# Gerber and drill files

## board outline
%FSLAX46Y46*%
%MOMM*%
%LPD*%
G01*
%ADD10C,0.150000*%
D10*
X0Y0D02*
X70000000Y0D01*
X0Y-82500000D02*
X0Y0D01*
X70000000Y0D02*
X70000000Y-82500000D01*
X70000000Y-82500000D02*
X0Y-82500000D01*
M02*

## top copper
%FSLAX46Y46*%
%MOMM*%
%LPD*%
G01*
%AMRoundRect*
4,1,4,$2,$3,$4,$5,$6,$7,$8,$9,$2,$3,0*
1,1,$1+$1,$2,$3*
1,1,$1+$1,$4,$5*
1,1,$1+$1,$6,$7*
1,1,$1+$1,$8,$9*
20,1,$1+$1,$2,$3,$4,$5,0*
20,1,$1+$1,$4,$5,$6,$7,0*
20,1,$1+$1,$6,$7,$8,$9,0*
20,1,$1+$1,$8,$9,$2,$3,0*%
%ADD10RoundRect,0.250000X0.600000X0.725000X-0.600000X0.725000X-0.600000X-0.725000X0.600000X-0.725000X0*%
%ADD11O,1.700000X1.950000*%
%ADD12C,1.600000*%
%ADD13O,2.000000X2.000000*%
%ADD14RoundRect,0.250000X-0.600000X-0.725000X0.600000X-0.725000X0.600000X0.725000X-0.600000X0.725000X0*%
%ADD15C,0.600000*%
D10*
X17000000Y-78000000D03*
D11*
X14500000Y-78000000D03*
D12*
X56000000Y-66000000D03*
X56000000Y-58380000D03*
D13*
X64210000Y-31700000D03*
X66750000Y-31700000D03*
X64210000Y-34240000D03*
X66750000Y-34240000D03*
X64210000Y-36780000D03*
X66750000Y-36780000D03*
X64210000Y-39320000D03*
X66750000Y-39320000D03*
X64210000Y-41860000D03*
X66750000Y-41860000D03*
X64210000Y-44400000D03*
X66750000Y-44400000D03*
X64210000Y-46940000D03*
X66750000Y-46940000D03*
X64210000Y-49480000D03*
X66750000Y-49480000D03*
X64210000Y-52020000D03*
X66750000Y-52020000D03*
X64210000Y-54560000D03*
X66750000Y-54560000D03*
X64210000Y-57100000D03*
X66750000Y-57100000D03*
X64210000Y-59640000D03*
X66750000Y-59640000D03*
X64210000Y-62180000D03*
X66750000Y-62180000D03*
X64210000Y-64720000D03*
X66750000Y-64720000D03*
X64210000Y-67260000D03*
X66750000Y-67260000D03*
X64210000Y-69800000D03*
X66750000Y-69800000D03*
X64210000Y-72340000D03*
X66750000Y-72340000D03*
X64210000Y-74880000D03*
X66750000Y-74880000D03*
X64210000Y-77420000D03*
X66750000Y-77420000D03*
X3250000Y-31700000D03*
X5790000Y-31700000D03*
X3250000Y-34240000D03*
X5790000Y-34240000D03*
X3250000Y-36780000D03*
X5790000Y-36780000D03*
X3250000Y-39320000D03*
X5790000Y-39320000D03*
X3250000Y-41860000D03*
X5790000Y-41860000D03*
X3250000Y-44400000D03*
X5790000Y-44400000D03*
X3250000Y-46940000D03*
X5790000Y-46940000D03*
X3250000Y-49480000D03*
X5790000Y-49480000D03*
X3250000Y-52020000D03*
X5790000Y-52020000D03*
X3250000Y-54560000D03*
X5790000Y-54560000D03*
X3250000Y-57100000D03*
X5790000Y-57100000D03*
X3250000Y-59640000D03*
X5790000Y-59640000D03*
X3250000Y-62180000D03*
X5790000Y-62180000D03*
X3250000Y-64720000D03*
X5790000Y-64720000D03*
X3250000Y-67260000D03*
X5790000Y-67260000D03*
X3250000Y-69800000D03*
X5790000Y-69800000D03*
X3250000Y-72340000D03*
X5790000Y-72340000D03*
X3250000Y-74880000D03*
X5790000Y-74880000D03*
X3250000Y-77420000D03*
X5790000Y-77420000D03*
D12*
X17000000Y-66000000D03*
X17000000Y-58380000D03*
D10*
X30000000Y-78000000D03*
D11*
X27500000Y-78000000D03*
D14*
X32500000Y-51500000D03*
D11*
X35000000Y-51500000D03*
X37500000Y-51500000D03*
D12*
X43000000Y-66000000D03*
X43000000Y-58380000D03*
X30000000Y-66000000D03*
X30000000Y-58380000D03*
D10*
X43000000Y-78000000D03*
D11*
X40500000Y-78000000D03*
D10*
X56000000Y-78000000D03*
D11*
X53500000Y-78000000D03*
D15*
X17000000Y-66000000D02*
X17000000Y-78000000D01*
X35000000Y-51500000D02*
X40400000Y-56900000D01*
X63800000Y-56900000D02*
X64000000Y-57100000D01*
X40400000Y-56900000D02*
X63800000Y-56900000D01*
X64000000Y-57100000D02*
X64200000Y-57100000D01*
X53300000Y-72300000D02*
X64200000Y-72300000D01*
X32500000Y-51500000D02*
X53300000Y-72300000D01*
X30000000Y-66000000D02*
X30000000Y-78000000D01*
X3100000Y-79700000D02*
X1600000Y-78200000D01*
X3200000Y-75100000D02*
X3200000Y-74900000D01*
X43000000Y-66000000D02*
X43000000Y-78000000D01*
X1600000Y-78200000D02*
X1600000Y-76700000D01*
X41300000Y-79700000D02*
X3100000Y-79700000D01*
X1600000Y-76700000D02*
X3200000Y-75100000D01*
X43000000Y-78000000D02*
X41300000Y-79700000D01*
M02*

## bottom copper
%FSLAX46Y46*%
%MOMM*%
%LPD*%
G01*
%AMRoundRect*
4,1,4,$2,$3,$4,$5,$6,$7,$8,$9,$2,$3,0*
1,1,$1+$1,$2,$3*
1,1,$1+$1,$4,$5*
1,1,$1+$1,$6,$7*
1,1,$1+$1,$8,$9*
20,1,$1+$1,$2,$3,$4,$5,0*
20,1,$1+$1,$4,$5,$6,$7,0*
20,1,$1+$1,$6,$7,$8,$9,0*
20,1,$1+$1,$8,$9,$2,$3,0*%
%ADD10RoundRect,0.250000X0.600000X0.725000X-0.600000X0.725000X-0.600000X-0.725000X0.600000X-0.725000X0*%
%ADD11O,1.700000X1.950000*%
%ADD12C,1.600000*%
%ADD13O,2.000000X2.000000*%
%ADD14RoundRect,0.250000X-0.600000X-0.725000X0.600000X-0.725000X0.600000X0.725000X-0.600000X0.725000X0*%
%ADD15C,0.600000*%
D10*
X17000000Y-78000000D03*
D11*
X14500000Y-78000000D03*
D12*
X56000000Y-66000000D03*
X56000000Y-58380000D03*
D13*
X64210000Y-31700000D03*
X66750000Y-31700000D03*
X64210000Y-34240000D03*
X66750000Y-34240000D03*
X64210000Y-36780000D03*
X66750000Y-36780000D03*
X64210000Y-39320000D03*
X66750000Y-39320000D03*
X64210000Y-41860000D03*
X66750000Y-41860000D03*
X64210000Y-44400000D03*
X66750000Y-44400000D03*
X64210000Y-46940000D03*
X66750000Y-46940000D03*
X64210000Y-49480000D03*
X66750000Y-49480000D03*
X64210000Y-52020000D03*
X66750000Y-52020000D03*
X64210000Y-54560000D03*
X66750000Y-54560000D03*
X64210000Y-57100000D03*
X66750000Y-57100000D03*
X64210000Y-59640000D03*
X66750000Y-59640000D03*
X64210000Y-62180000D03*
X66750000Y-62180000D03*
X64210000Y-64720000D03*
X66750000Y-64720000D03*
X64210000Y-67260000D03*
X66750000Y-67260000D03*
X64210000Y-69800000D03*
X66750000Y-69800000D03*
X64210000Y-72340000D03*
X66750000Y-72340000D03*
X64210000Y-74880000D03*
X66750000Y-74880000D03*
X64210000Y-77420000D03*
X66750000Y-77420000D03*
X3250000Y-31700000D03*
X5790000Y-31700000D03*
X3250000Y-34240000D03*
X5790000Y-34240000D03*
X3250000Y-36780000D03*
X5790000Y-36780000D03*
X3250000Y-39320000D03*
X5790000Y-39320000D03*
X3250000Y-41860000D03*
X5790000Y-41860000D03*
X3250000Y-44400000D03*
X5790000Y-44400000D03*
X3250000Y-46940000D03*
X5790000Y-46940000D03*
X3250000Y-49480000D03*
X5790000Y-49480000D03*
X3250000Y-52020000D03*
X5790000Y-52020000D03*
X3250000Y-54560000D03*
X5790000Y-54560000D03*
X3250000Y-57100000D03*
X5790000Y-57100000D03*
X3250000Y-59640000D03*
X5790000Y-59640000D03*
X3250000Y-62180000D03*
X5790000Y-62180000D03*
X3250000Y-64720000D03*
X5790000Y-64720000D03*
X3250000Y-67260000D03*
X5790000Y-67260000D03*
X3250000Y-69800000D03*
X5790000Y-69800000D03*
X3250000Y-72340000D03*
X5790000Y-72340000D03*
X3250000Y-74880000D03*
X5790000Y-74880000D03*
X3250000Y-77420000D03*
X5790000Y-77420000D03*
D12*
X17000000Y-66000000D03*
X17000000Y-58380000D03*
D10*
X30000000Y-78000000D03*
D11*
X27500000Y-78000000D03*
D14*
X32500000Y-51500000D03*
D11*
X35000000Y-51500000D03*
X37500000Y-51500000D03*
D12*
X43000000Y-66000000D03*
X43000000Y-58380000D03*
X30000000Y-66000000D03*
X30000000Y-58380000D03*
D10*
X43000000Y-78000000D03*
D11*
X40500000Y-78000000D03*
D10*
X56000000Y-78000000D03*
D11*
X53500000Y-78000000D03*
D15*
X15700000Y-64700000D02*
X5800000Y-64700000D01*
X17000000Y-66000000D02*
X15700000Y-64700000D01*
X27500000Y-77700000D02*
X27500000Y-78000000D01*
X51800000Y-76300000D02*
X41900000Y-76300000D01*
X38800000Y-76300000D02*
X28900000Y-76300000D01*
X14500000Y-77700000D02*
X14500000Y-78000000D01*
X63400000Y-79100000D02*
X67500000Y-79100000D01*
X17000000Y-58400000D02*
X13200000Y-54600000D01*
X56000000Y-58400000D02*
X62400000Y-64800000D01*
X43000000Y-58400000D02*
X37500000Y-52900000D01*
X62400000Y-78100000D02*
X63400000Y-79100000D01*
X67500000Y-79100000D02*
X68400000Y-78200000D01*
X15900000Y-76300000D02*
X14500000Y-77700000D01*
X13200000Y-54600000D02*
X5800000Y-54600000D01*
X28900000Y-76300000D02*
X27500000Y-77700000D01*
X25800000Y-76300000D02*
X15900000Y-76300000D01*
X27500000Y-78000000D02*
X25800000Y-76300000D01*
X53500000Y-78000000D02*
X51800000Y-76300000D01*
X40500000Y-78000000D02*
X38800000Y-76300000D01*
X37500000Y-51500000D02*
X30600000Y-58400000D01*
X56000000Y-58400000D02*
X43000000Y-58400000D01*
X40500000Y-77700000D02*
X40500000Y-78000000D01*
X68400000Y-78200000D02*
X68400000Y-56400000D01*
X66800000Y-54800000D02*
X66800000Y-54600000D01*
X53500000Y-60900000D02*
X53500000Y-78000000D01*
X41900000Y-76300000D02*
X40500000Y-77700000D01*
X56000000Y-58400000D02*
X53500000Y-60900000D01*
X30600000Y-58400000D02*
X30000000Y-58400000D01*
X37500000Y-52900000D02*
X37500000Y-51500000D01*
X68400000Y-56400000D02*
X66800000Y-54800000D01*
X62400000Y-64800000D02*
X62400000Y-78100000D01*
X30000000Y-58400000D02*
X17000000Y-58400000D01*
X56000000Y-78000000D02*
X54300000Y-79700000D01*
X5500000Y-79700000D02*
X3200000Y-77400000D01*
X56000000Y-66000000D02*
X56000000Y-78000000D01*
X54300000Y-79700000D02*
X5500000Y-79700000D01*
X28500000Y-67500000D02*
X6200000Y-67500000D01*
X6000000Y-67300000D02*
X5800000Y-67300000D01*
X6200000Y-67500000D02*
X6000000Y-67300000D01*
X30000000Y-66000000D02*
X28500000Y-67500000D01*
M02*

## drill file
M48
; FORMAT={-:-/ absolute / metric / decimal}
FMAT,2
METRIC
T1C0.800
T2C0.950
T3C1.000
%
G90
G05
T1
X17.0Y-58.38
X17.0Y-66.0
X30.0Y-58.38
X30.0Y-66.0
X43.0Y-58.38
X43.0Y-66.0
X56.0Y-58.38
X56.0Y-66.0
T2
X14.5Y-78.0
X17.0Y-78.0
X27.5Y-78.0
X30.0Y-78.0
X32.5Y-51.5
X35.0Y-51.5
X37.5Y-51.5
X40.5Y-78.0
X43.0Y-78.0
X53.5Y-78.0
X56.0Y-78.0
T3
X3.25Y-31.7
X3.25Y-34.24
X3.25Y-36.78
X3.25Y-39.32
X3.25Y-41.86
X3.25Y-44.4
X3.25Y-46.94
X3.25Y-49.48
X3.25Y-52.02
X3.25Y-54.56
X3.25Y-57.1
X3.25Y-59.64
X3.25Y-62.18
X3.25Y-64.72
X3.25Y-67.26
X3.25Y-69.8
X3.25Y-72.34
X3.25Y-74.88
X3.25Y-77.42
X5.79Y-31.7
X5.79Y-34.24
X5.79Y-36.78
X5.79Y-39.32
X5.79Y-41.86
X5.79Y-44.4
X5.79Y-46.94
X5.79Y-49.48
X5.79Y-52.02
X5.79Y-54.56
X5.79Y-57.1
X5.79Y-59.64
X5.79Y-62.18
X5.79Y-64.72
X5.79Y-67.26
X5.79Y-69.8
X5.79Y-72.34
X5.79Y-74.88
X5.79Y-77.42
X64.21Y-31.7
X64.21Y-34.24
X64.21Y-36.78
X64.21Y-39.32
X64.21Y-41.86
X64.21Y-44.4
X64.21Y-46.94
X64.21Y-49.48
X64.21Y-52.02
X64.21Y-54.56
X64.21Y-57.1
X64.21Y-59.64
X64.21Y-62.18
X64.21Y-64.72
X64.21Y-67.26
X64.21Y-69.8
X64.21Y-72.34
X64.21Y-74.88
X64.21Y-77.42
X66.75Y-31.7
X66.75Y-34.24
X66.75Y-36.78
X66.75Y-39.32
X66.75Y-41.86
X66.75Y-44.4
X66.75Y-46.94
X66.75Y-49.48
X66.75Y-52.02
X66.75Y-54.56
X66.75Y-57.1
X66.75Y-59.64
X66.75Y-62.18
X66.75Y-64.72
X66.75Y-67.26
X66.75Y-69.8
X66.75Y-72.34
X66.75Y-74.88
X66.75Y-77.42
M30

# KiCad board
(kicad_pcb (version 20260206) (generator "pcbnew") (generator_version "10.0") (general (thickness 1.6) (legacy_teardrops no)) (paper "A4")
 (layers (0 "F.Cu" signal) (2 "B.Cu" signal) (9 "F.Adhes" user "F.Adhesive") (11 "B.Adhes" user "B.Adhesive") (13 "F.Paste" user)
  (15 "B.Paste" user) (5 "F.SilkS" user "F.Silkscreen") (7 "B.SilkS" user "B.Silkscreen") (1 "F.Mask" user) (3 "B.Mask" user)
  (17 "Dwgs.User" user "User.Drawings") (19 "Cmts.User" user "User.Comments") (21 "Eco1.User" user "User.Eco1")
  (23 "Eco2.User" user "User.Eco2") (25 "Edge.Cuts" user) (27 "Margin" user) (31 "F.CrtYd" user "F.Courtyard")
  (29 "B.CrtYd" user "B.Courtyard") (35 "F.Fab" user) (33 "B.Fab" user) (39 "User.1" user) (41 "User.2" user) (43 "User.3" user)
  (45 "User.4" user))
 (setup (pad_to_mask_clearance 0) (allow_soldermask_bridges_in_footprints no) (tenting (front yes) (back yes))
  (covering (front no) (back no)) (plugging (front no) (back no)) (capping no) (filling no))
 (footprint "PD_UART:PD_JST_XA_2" (layer "F.Cu") (at 17 78 180)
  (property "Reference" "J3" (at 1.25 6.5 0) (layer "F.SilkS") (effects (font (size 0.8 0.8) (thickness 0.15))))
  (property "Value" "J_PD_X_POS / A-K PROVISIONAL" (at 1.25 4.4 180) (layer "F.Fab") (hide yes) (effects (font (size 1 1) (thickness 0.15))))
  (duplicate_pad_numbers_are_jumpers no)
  (pad "1" thru_hole roundrect (at 0 0 180) (size 1.7 1.95) (drill 0.95) (layers "*.Cu" "*.Mask") (remove_unused_layers no)
   (roundrect_rratio 0.147059) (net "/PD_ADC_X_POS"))
  (pad "2" thru_hole oval (at 2.5 0 180) (size 1.7 1.95) (drill 0.95) (layers "*.Cu" "*.Mask") (remove_unused_layers no) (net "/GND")))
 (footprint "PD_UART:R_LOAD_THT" (layer "F.Cu") (at 56 66 90)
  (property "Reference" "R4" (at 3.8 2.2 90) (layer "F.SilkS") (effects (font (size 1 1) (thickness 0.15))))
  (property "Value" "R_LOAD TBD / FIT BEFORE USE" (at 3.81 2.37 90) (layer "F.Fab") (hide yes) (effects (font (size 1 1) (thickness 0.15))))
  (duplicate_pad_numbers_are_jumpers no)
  (pad "1" thru_hole circle (at 0 0 90) (size 1.6 1.6) (drill 0.8) (layers "*.Cu" "*.Mask") (remove_unused_layers no) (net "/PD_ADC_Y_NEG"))
  (pad "2" thru_hole circle (at 7.62 0 90) (size 1.6 1.6) (drill 0.8) (layers "*.Cu" "*.Mask") (remove_unused_layers no) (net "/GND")))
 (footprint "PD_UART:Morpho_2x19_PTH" (layer "F.Cu") (at 64.21 31.7)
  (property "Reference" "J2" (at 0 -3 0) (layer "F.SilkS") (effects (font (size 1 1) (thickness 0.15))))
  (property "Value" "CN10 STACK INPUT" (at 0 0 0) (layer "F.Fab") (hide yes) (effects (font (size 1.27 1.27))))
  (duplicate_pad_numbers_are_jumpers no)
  (pad "1" thru_hole oval (at 0 0) (size 2 2) (drill 1) (layers "*.Cu") (remove_unused_layers no) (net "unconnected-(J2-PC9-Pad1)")
   (thermal_bridge_angle 45))
  (pad "2" thru_hole oval (at 2.54 0) (size 2 2) (drill 1) (layers "*.Cu") (remove_unused_layers no) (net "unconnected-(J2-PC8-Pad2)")
   (thermal_bridge_angle 45))
  (pad "3" thru_hole oval (at 0 2.54) (size 2 2) (drill 1) (layers "*.Cu") (remove_unused_layers no) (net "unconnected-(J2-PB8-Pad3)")
   (thermal_bridge_angle 45))
  (pad "4" thru_hole oval (at 2.54 2.54) (size 2 2) (drill 1) (layers "*.Cu") (remove_unused_layers no) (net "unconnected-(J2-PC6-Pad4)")
   (thermal_bridge_angle 45))
  (pad "5" thru_hole oval (at 0 5.08) (size 2 2) (drill 1) (layers "*.Cu") (remove_unused_layers no) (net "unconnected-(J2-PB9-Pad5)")
   (thermal_bridge_angle 45))
  (pad "6" thru_hole oval (at 2.54 5.08) (size 2 2) (drill 1) (layers "*.Cu") (remove_unused_layers no) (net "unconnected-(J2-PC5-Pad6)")
   (thermal_bridge_angle 45))
  (pad "7" thru_hole oval (at 0 7.62) (size 2 2) (drill 1) (layers "*.Cu") (remove_unused_layers no) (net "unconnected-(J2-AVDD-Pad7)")
   (thermal_bridge_angle 45))
  (pad "8" thru_hole oval (at 2.54 7.62) (size 2 2) (drill 1) (layers "*.Cu") (remove_unused_layers no) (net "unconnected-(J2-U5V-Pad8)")
   (thermal_bridge_angle 45))
  (pad "9" thru_hole oval (at 0 10.16) (size 2 2) (drill 1) (layers "*.Cu") (remove_unused_layers no) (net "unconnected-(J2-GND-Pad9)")
   (thermal_bridge_angle 45))
  (pad "10" thru_hole oval (at 2.54 10.16) (size 2 2) (drill 1) (layers "*.Cu") (remove_unused_layers no) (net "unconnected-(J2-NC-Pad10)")
   (thermal_bridge_angle 45))
  (pad "11" thru_hole oval (at 0 12.7) (size 2 2) (drill 1) (layers "*.Cu") (remove_unused_layers no) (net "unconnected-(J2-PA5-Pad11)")
   (thermal_bridge_angle 45))
  (pad "12" thru_hole oval (at 2.54 12.7) (size 2 2) (drill 1) (layers "*.Cu") (remove_unused_layers no) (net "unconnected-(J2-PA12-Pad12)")
   (thermal_bridge_angle 45))
  (pad "13" thru_hole oval (at 0 15.24) (size 2 2) (drill 1) (layers "*.Cu") (remove_unused_layers no) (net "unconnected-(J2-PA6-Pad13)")
   (thermal_bridge_angle 45))
  (pad "14" thru_hole oval (at 2.54 15.24) (size 2 2) (drill 1) (layers "*.Cu") (remove_unused_layers no)
   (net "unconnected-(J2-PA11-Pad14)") (thermal_bridge_angle 45))
  (pad "15" thru_hole oval (at 0 17.78) (size 2 2) (drill 1) (layers "*.Cu") (remove_unused_layers no) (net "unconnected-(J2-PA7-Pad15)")
   (thermal_bridge_angle 45))
  (pad "16" thru_hole oval (at 2.54 17.78) (size 2 2) (drill 1) (layers "*.Cu") (remove_unused_layers no)
   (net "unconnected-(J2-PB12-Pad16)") (thermal_bridge_angle 45))
  (pad "17" thru_hole oval (at 0 20.32) (size 2 2) (drill 1) (layers "*.Cu") (remove_unused_layers no) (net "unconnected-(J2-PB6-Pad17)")
   (thermal_bridge_angle 45))
  (pad "18" thru_hole oval (at 2.54 20.32) (size 2 2) (drill 1) (layers "*.Cu") (remove_unused_layers no)
   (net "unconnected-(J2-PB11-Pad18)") (thermal_bridge_angle 45))
  (pad "19" thru_hole oval (at 0 22.86) (size 2 2) (drill 1) (layers "*.Cu") (remove_unused_layers no) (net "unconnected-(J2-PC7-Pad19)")
   (thermal_bridge_angle 45))
  (pad "20" thru_hole oval (at 2.54 22.86) (size 2 2) (drill 1) (layers "*.Cu") (remove_unused_layers no) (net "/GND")
   (thermal_bridge_angle 45))
  (pad "21" thru_hole oval (at 0 25.4) (size 2 2) (drill 1) (layers "*.Cu") (remove_unused_layers no) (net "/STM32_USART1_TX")
   (thermal_bridge_angle 45))
  (pad "22" thru_hole oval (at 2.54 25.4) (size 2 2) (drill 1) (layers "*.Cu") (remove_unused_layers no) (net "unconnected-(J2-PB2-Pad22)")
   (thermal_bridge_angle 45))
  (pad "23" thru_hole oval (at 0 27.94) (size 2 2) (drill 1) (layers "*.Cu") (remove_unused_layers no) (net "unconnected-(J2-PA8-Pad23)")
   (thermal_bridge_angle 45))
  (pad "24" thru_hole oval (at 2.54 27.94) (size 2 2) (drill 1) (layers "*.Cu") (remove_unused_layers no) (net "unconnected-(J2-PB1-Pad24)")
   (thermal_bridge_angle 45))
  (pad "25" thru_hole oval (at 0 30.48) (size 2 2) (drill 1) (layers "*.Cu") (remove_unused_layers no) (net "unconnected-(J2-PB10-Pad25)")
   (thermal_bridge_angle 45))
  (pad "26" thru_hole oval (at 2.54 30.48) (size 2 2) (drill 1) (layers "*.Cu") (remove_unused_layers no)
   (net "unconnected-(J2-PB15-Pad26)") (thermal_bridge_angle 45))
  (pad "27" thru_hole oval (at 0 33.02) (size 2 2) (drill 1) (layers "*.Cu") (remove_unused_layers no) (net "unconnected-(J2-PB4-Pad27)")
   (thermal_bridge_angle 45))
  (pad "28" thru_hole oval (at 2.54 33.02) (size 2 2) (drill 1) (layers "*.Cu") (remove_unused_layers no)
   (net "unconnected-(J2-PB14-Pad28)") (thermal_bridge_angle 45))
  (pad "29" thru_hole oval (at 0 35.56) (size 2 2) (drill 1) (layers "*.Cu") (remove_unused_layers no) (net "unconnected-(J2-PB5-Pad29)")
   (thermal_bridge_angle 45))
  (pad "30" thru_hole oval (at 2.54 35.56) (size 2 2) (drill 1) (layers "*.Cu") (remove_unused_layers no)
   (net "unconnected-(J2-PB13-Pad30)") (thermal_bridge_angle 45))
  (pad "31" thru_hole oval (at 0 38.1) (size 2 2) (drill 1) (layers "*.Cu") (remove_unused_layers no) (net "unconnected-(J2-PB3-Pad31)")
   (thermal_bridge_angle 45))
  (pad "32" thru_hole oval (at 2.54 38.1) (size 2 2) (drill 1) (layers "*.Cu") (remove_unused_layers no) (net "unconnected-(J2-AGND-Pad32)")
   (thermal_bridge_angle 45))
  (pad "33" thru_hole oval (at 0 40.64) (size 2 2) (drill 1) (layers "*.Cu") (remove_unused_layers no) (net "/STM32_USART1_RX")
   (thermal_bridge_angle 45))
  (pad "34" thru_hole oval (at 2.54 40.64) (size 2 2) (drill 1) (layers "*.Cu") (remove_unused_layers no) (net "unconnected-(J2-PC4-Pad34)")
   (thermal_bridge_angle 45))
  (pad "35" thru_hole oval (at 0 43.18) (size 2 2) (drill 1) (layers "*.Cu") (remove_unused_layers no) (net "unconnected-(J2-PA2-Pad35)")
   (thermal_bridge_angle 45))
  (pad "36" thru_hole oval (at 2.54 43.18) (size 2 2) (drill 1) (layers "*.Cu") (remove_unused_layers no) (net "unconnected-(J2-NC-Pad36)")
   (thermal_bridge_angle 45))
  (pad "37" thru_hole oval (at 0 45.72) (size 2 2) (drill 1) (layers "*.Cu") (remove_unused_layers no) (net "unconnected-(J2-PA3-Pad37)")
   (thermal_bridge_angle 45))
  (pad "38" thru_hole oval (at 2.54 45.72) (size 2 2) (drill 1) (layers "*.Cu") (remove_unused_layers no) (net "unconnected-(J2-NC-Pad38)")
   (thermal_bridge_angle 45)))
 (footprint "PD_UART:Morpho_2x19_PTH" (layer "F.Cu") (at 3.25 31.7)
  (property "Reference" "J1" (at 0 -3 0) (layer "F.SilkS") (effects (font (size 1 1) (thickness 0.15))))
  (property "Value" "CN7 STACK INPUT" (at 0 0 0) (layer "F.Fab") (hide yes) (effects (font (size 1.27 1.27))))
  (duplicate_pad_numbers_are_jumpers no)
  (pad "1" thru_hole oval (at 0 0) (size 2 2) (drill 1) (layers "*.Cu") (remove_unused_layers no) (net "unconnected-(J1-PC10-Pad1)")
   (thermal_bridge_angle 45))
  (pad "2" thru_hole oval (at 2.54 0) (size 2 2) (drill 1) (layers "*.Cu") (remove_unused_layers no) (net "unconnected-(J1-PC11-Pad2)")
   (thermal_bridge_angle 45))
  (pad "3" thru_hole oval (at 0 2.54) (size 2 2) (drill 1) (layers "*.Cu") (remove_unused_layers no) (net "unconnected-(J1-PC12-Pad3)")
   (thermal_bridge_angle 45))
  (pad "4" thru_hole oval (at 2.54 2.54) (size 2 2) (drill 1) (layers "*.Cu") (remove_unused_layers no) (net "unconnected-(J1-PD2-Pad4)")
   (thermal_bridge_angle 45))
  (pad "5" thru_hole oval (at 0 5.08) (size 2 2) (drill 1) (layers "*.Cu") (remove_unused_layers no) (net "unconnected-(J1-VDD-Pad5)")
   (thermal_bridge_angle 45))
  (pad "6" thru_hole oval (at 2.54 5.08) (size 2 2) (drill 1) (layers "*.Cu") (remove_unused_layers no) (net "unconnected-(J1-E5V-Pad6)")
   (thermal_bridge_angle 45))
  (pad "7" thru_hole oval (at 0 7.62) (size 2 2) (drill 1) (layers "*.Cu") (remove_unused_layers no) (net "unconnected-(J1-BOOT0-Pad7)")
   (thermal_bridge_angle 45))
  (pad "8" thru_hole oval (at 2.54 7.62) (size 2 2) (drill 1) (layers "*.Cu") (remove_unused_layers no) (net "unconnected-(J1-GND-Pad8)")
   (thermal_bridge_angle 45))
  (pad "9" thru_hole oval (at 0 10.16) (size 2 2) (drill 1) (layers "*.Cu") (remove_unused_layers no) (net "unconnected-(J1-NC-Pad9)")
   (thermal_bridge_angle 45))
  (pad "10" thru_hole oval (at 2.54 10.16) (size 2 2) (drill 1) (layers "*.Cu") (remove_unused_layers no) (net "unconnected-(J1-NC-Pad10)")
   (thermal_bridge_angle 45))
  (pad "11" thru_hole oval (at 0 12.7) (size 2 2) (drill 1) (layers "*.Cu") (remove_unused_layers no) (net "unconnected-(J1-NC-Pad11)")
   (thermal_bridge_angle 45))
  (pad "12" thru_hole oval (at 2.54 12.7) (size 2 2) (drill 1) (layers "*.Cu") (remove_unused_layers no)
   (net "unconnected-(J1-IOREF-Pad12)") (thermal_bridge_angle 45))
  (pad "13" thru_hole oval (at 0 15.24) (size 2 2) (drill 1) (layers "*.Cu") (remove_unused_layers no) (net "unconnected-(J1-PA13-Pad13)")
   (thermal_bridge_angle 45))
  (pad "14" thru_hole oval (at 2.54 15.24) (size 2 2) (drill 1) (layers "*.Cu") (remove_unused_layers no)
   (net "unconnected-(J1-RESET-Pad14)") (thermal_bridge_angle 45))
  (pad "15" thru_hole oval (at 0 17.78) (size 2 2) (drill 1) (layers "*.Cu") (remove_unused_layers no) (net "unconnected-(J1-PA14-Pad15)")
   (thermal_bridge_angle 45))
  (pad "16" thru_hole oval (at 2.54 17.78) (size 2 2) (drill 1) (layers "*.Cu") (remove_unused_layers no) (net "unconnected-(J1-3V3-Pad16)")
   (thermal_bridge_angle 45))
  (pad "17" thru_hole oval (at 0 20.32) (size 2 2) (drill 1) (layers "*.Cu") (remove_unused_layers no) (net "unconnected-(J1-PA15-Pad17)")
   (thermal_bridge_angle 45))
  (pad "18" thru_hole oval (at 2.54 20.32) (size 2 2) (drill 1) (layers "*.Cu") (remove_unused_layers no) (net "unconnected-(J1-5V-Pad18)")
   (thermal_bridge_angle 45))
  (pad "19" thru_hole oval (at 0 22.86) (size 2 2) (drill 1) (layers "*.Cu") (remove_unused_layers no) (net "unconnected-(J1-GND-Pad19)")
   (thermal_bridge_angle 45))
  (pad "20" thru_hole oval (at 2.54 22.86) (size 2 2) (drill 1) (layers "*.Cu") (remove_unused_layers no) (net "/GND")
   (thermal_bridge_angle 45))
  (pad "21" thru_hole oval (at 0 25.4) (size 2 2) (drill 1) (layers "*.Cu") (remove_unused_layers no) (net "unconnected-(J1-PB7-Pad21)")
   (thermal_bridge_angle 45))
  (pad "22" thru_hole oval (at 2.54 25.4) (size 2 2) (drill 1) (layers "*.Cu") (remove_unused_layers no) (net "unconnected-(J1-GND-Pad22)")
   (thermal_bridge_angle 45))
  (pad "23" thru_hole oval (at 0 27.94) (size 2 2) (drill 1) (layers "*.Cu") (remove_unused_layers no) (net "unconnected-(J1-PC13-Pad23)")
   (thermal_bridge_angle 45))
  (pad "24" thru_hole oval (at 2.54 27.94) (size 2 2) (drill 1) (layers "*.Cu") (remove_unused_layers no) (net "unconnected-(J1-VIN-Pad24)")
   (thermal_bridge_angle 45))
  (pad "25" thru_hole oval (at 0 30.48) (size 2 2) (drill 1) (layers "*.Cu") (remove_unused_layers no) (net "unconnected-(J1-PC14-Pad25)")
   (thermal_bridge_angle 45))
  (pad "26" thru_hole oval (at 2.54 30.48) (size 2 2) (drill 1) (layers "*.Cu") (remove_unused_layers no) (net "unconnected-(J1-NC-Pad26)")
   (thermal_bridge_angle 45))
  (pad "27" thru_hole oval (at 0 33.02) (size 2 2) (drill 1) (layers "*.Cu") (remove_unused_layers no) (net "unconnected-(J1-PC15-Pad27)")
   (thermal_bridge_angle 45))
  (pad "28" thru_hole oval (at 2.54 33.02) (size 2 2) (drill 1) (layers "*.Cu") (remove_unused_layers no) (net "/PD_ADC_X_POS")
   (thermal_bridge_angle 45))
  (pad "29" thru_hole oval (at 0 35.56) (size 2 2) (drill 1) (layers "*.Cu") (remove_unused_layers no) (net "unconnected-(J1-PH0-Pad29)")
   (thermal_bridge_angle 45))
  (pad "30" thru_hole oval (at 2.54 35.56) (size 2 2) (drill 1) (layers "*.Cu") (remove_unused_layers no) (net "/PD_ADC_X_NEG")
   (thermal_bridge_angle 45))
  (pad "31" thru_hole oval (at 0 38.1) (size 2 2) (drill 1) (layers "*.Cu") (remove_unused_layers no) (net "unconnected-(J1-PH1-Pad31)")
   (thermal_bridge_angle 45))
  (pad "32" thru_hole oval (at 2.54 38.1) (size 2 2) (drill 1) (layers "*.Cu") (remove_unused_layers no) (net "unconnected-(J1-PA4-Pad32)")
   (thermal_bridge_angle 45))
  (pad "33" thru_hole oval (at 0 40.64) (size 2 2) (drill 1) (layers "*.Cu") (remove_unused_layers no) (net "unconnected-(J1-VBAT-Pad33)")
   (thermal_bridge_angle 45))
  (pad "34" thru_hole oval (at 2.54 40.64) (size 2 2) (drill 1) (layers "*.Cu") (remove_unused_layers no) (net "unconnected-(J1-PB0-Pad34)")
   (thermal_bridge_angle 45))
  (pad "35" thru_hole oval (at 0 43.18) (size 2 2) (drill 1) (layers "*.Cu") (remove_unused_layers no) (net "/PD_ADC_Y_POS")
   (thermal_bridge_angle 45))
  (pad "36" thru_hole oval (at 2.54 43.18) (size 2 2) (drill 1) (layers "*.Cu") (remove_unused_layers no)
   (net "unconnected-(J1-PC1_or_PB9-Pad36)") (thermal_bridge_angle 45))
  (pad "37" thru_hole oval (at 0 45.72) (size 2 2) (drill 1) (layers "*.Cu") (remove_unused_layers no) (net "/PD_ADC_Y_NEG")
   (thermal_bridge_angle 45))
  (pad "38" thru_hole oval (at 2.54 45.72) (size 2 2) (drill 1) (layers "*.Cu") (remove_unused_layers no) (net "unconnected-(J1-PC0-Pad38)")
   (thermal_bridge_angle 45)))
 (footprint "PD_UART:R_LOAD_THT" (layer "F.Cu") (at 17 66 90)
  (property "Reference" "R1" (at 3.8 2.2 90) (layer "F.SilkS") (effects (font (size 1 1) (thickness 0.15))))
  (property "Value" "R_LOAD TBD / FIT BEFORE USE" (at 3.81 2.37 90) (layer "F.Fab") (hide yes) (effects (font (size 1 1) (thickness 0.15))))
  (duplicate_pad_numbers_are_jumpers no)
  (pad "1" thru_hole circle (at 0 0 90) (size 1.6 1.6) (drill 0.8) (layers "*.Cu" "*.Mask") (remove_unused_layers no) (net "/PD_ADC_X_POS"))
  (pad "2" thru_hole circle (at 7.62 0 90) (size 1.6 1.6) (drill 0.8) (layers "*.Cu" "*.Mask") (remove_unused_layers no) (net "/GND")))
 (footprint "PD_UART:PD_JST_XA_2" (layer "F.Cu") (at 30 78 180)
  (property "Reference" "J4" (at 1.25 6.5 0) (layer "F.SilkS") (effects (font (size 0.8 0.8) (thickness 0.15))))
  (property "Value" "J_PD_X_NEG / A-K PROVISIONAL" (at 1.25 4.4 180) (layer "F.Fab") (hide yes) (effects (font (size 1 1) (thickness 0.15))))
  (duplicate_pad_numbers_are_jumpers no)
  (pad "1" thru_hole roundrect (at 0 0 180) (size 1.7 1.95) (drill 0.95) (layers "*.Cu" "*.Mask") (remove_unused_layers no)
   (roundrect_rratio 0.147059) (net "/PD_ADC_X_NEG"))
  (pad "2" thru_hole oval (at 2.5 0 180) (size 1.7 1.95) (drill 0.95) (layers "*.Cu" "*.Mask") (remove_unused_layers no) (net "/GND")))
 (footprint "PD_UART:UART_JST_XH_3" (layer "F.Cu") (at 32.5 51.5)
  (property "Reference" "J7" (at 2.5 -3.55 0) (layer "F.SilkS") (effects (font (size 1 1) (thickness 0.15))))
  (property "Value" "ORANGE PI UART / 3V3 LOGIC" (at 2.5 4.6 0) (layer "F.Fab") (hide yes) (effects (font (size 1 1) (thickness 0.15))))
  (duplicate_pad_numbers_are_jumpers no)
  (pad "1" thru_hole roundrect (at 0 0) (size 1.7 1.95) (drill 0.95) (layers "*.Cu" "*.Mask") (remove_unused_layers no)
   (roundrect_rratio 0.147059) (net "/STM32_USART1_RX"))
  (pad "2" thru_hole oval (at 2.5 0) (size 1.7 1.95) (drill 0.95) (layers "*.Cu" "*.Mask") (remove_unused_layers no)
   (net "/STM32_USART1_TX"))
  (pad "3" thru_hole oval (at 5 0) (size 1.7 1.95) (drill 0.95) (layers "*.Cu" "*.Mask") (remove_unused_layers no) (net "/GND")))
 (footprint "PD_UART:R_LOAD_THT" (layer "F.Cu") (at 43 66 90)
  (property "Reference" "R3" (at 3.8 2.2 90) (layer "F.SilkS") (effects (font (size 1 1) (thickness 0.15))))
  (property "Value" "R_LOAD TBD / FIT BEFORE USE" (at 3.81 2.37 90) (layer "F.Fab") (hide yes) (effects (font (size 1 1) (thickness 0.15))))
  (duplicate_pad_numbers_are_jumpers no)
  (pad "1" thru_hole circle (at 0 0 90) (size 1.6 1.6) (drill 0.8) (layers "*.Cu" "*.Mask") (remove_unused_layers no) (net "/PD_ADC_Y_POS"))
  (pad "2" thru_hole circle (at 7.62 0 90) (size 1.6 1.6) (drill 0.8) (layers "*.Cu" "*.Mask") (remove_unused_layers no) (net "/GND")))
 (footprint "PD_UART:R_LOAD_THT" (layer "F.Cu") (at 30 66 90)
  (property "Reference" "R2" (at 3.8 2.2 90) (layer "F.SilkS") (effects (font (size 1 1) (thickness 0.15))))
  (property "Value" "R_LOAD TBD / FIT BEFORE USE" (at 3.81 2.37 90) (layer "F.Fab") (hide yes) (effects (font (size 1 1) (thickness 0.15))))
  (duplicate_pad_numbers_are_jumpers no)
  (pad "1" thru_hole circle (at 0 0 90) (size 1.6 1.6) (drill 0.8) (layers "*.Cu" "*.Mask") (remove_unused_layers no) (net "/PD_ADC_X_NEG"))
  (pad "2" thru_hole circle (at 7.62 0 90) (size 1.6 1.6) (drill 0.8) (layers "*.Cu" "*.Mask") (remove_unused_layers no) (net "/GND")))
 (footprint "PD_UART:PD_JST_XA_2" (layer "F.Cu") (at 43 78 180)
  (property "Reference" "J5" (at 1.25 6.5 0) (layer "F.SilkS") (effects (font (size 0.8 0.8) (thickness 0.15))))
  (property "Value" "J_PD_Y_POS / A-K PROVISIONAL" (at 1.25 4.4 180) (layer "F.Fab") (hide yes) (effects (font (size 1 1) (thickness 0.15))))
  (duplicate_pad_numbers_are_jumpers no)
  (pad "1" thru_hole roundrect (at 0 0 180) (size 1.7 1.95) (drill 0.95) (layers "*.Cu" "*.Mask") (remove_unused_layers no)
   (roundrect_rratio 0.147059) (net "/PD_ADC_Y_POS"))
  (pad "2" thru_hole oval (at 2.5 0 180) (size 1.7 1.95) (drill 0.95) (layers "*.Cu" "*.Mask") (remove_unused_layers no) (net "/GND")))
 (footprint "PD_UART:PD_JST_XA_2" (layer "F.Cu") (at 56 78 180)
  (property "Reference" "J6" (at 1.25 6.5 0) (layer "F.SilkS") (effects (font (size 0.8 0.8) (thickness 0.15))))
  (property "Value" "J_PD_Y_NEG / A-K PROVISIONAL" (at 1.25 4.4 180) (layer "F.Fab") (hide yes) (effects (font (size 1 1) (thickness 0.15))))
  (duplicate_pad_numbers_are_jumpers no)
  (pad "1" thru_hole roundrect (at 0 0 180) (size 1.7 1.95) (drill 0.95) (layers "*.Cu" "*.Mask") (remove_unused_layers no)
   (roundrect_rratio 0.147059) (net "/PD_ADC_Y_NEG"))
  (pad "2" thru_hole oval (at 2.5 0 180) (size 1.7 1.95) (drill 0.95) (layers "*.Cu" "*.Mask") (remove_unused_layers no) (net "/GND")))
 (gr_line (start 0 0) (end 70 0) (stroke (width 0.15) (type default)) (layer "Edge.Cuts"))
 (gr_line (start 0 82.5) (end 0 0) (stroke (width 0.15) (type default)) (layer "Edge.Cuts"))
 (gr_line (start 70 0) (end 70 82.5) (stroke (width 0.15) (type default)) (layer "Edge.Cuts"))
 (gr_line (start 70 82.5) (end 0 82.5) (stroke (width 0.15) (type default)) (layer "Edge.Cuts"))
 (segment (start 17 66) (end 17 78) (width 0.6) (layer "F.Cu") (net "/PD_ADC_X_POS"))
 (segment (start 15.7 64.7) (end 5.8 64.7) (width 0.6) (layer "B.Cu") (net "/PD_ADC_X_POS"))
 (segment (start 17 66) (end 15.7 64.7) (width 0.6) (layer "B.Cu") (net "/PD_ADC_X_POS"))
 (segment (start 27.5 77.7) (end 27.5 78) (width 0.6) (layer "B.Cu") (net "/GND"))
 (segment (start 51.8 76.3) (end 41.9 76.3) (width 0.6) (layer "B.Cu") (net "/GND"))
 (segment (start 38.8 76.3) (end 28.9 76.3) (width 0.6) (layer "B.Cu") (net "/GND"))
 (segment (start 14.5 77.7) (end 14.5 78) (width 0.6) (layer "B.Cu") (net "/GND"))
 (segment (start 63.4 79.1) (end 67.5 79.1) (width 0.6) (layer "B.Cu") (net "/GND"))
 (segment (start 17 58.4) (end 13.2 54.6) (width 0.6) (layer "B.Cu") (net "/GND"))
 (segment (start 56 58.4) (end 62.4 64.8) (width 0.6) (layer "B.Cu") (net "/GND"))
 (segment (start 43 58.4) (end 37.5 52.9) (width 0.6) (layer "B.Cu") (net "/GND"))
 (segment (start 62.4 78.1) (end 63.4 79.1) (width 0.6) (layer "B.Cu") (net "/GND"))
 (segment (start 67.5 79.1) (end 68.4 78.2) (width 0.6) (layer "B.Cu") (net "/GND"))
 (segment (start 15.9 76.3) (end 14.5 77.7) (width 0.6) (layer "B.Cu") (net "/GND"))
 (segment (start 13.2 54.6) (end 5.8 54.6) (width 0.6) (layer "B.Cu") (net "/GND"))
 (segment (start 28.9 76.3) (end 27.5 77.7) (width 0.6) (layer "B.Cu") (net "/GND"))
 (segment (start 25.8 76.3) (end 15.9 76.3) (width 0.6) (layer "B.Cu") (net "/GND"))
 (segment (start 27.5 78) (end 25.8 76.3) (width 0.6) (layer "B.Cu") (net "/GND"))
 (segment (start 53.5 78) (end 51.8 76.3) (width 0.6) (layer "B.Cu") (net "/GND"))
 (segment (start 40.5 78) (end 38.8 76.3) (width 0.6) (layer "B.Cu") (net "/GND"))
 (segment (start 37.5 51.5) (end 30.6 58.4) (width 0.6) (layer "B.Cu") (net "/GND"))
 (segment (start 56 58.4) (end 43 58.4) (width 0.6) (layer "B.Cu") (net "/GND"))
 (segment (start 40.5 77.7) (end 40.5 78) (width 0.6) (layer "B.Cu") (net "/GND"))
 (segment (start 68.4 78.2) (end 68.4 56.4) (width 0.6) (layer "B.Cu") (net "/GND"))
 (segment (start 66.8 54.8) (end 66.8 54.6) (width 0.6) (layer "B.Cu") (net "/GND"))
 (segment (start 53.5 60.9) (end 53.5 78) (width 0.6) (layer "B.Cu") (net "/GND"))
 (segment (start 41.9 76.3) (end 40.5 77.7) (width 0.6) (layer "B.Cu") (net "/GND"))
 (segment (start 56 58.4) (end 53.5 60.9) (width 0.6) (layer "B.Cu") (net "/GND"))
 (segment (start 30.6 58.4) (end 30 58.4) (width 0.6) (layer "B.Cu") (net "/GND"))
 (segment (start 37.5 52.9) (end 37.5 51.5) (width 0.6) (layer "B.Cu") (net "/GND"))
 (segment (start 68.4 56.4) (end 66.8 54.8) (width 0.6) (layer "B.Cu") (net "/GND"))
 (segment (start 62.4 64.8) (end 62.4 78.1) (width 0.6) (layer "B.Cu") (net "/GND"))
 (segment (start 30 58.4) (end 17 58.4) (width 0.6) (layer "B.Cu") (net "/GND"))
 (segment (start 56 78) (end 54.3 79.7) (width 0.6) (layer "B.Cu") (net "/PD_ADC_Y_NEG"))
 (segment (start 5.5 79.7) (end 3.2 77.4) (width 0.6) (layer "B.Cu") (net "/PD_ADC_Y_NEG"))
 (segment (start 56 66) (end 56 78) (width 0.6) (layer "B.Cu") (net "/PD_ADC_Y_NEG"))
 (segment (start 54.3 79.7) (end 5.5 79.7) (width 0.6) (layer "B.Cu") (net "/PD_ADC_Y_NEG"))
 (segment (start 35 51.5) (end 40.4 56.9) (width 0.6) (layer "F.Cu") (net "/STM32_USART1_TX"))
 (segment (start 63.8 56.9) (end 64 57.1) (width 0.6) (layer "F.Cu") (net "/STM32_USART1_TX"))
 (segment (start 40.4 56.9) (end 63.8 56.9) (width 0.6) (layer "F.Cu") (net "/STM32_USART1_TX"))
 (segment (start 64 57.1) (end 64.2 57.1) (width 0.6) (layer "F.Cu") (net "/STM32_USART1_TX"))
 (segment (start 53.3 72.3) (end 64.2 72.3) (width 0.6) (layer "F.Cu") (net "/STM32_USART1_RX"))
 (segment (start 32.5 51.5) (end 53.3 72.3) (width 0.6) (layer "F.Cu") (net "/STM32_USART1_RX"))
 (segment (start 30 66) (end 30 78) (width 0.6) (layer "F.Cu") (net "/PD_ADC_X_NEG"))
 (segment (start 28.5 67.5) (end 6.2 67.5) (width 0.6) (layer "B.Cu") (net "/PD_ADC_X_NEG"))
 (segment (start 6 67.3) (end 5.8 67.3) (width 0.6) (layer "B.Cu") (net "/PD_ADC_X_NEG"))
 (segment (start 6.2 67.5) (end 6 67.3) (width 0.6) (layer "B.Cu") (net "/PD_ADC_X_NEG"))
 (segment (start 30 66) (end 28.5 67.5) (width 0.6) (layer "B.Cu") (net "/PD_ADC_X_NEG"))
 (segment (start 3.1 79.7) (end 1.6 78.2) (width 0.6) (layer "F.Cu") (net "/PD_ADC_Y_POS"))
 (segment (start 3.2 75.1) (end 3.2 74.9) (width 0.6) (layer "F.Cu") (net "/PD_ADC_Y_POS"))
 (segment (start 43 66) (end 43 78) (width 0.6) (layer "F.Cu") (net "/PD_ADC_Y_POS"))
 (segment (start 1.6 78.2) (end 1.6 76.7) (width 0.6) (layer "F.Cu") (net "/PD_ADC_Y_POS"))
 (segment (start 41.3 79.7) (end 3.1 79.7) (width 0.6) (layer "F.Cu") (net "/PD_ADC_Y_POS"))
 (segment (start 1.6 76.7) (end 3.2 75.1) (width 0.6) (layer "F.Cu") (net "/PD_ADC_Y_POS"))
 (segment (start 43 78) (end 41.3 79.7) (width 0.6) (layer "F.Cu") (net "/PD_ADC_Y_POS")))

